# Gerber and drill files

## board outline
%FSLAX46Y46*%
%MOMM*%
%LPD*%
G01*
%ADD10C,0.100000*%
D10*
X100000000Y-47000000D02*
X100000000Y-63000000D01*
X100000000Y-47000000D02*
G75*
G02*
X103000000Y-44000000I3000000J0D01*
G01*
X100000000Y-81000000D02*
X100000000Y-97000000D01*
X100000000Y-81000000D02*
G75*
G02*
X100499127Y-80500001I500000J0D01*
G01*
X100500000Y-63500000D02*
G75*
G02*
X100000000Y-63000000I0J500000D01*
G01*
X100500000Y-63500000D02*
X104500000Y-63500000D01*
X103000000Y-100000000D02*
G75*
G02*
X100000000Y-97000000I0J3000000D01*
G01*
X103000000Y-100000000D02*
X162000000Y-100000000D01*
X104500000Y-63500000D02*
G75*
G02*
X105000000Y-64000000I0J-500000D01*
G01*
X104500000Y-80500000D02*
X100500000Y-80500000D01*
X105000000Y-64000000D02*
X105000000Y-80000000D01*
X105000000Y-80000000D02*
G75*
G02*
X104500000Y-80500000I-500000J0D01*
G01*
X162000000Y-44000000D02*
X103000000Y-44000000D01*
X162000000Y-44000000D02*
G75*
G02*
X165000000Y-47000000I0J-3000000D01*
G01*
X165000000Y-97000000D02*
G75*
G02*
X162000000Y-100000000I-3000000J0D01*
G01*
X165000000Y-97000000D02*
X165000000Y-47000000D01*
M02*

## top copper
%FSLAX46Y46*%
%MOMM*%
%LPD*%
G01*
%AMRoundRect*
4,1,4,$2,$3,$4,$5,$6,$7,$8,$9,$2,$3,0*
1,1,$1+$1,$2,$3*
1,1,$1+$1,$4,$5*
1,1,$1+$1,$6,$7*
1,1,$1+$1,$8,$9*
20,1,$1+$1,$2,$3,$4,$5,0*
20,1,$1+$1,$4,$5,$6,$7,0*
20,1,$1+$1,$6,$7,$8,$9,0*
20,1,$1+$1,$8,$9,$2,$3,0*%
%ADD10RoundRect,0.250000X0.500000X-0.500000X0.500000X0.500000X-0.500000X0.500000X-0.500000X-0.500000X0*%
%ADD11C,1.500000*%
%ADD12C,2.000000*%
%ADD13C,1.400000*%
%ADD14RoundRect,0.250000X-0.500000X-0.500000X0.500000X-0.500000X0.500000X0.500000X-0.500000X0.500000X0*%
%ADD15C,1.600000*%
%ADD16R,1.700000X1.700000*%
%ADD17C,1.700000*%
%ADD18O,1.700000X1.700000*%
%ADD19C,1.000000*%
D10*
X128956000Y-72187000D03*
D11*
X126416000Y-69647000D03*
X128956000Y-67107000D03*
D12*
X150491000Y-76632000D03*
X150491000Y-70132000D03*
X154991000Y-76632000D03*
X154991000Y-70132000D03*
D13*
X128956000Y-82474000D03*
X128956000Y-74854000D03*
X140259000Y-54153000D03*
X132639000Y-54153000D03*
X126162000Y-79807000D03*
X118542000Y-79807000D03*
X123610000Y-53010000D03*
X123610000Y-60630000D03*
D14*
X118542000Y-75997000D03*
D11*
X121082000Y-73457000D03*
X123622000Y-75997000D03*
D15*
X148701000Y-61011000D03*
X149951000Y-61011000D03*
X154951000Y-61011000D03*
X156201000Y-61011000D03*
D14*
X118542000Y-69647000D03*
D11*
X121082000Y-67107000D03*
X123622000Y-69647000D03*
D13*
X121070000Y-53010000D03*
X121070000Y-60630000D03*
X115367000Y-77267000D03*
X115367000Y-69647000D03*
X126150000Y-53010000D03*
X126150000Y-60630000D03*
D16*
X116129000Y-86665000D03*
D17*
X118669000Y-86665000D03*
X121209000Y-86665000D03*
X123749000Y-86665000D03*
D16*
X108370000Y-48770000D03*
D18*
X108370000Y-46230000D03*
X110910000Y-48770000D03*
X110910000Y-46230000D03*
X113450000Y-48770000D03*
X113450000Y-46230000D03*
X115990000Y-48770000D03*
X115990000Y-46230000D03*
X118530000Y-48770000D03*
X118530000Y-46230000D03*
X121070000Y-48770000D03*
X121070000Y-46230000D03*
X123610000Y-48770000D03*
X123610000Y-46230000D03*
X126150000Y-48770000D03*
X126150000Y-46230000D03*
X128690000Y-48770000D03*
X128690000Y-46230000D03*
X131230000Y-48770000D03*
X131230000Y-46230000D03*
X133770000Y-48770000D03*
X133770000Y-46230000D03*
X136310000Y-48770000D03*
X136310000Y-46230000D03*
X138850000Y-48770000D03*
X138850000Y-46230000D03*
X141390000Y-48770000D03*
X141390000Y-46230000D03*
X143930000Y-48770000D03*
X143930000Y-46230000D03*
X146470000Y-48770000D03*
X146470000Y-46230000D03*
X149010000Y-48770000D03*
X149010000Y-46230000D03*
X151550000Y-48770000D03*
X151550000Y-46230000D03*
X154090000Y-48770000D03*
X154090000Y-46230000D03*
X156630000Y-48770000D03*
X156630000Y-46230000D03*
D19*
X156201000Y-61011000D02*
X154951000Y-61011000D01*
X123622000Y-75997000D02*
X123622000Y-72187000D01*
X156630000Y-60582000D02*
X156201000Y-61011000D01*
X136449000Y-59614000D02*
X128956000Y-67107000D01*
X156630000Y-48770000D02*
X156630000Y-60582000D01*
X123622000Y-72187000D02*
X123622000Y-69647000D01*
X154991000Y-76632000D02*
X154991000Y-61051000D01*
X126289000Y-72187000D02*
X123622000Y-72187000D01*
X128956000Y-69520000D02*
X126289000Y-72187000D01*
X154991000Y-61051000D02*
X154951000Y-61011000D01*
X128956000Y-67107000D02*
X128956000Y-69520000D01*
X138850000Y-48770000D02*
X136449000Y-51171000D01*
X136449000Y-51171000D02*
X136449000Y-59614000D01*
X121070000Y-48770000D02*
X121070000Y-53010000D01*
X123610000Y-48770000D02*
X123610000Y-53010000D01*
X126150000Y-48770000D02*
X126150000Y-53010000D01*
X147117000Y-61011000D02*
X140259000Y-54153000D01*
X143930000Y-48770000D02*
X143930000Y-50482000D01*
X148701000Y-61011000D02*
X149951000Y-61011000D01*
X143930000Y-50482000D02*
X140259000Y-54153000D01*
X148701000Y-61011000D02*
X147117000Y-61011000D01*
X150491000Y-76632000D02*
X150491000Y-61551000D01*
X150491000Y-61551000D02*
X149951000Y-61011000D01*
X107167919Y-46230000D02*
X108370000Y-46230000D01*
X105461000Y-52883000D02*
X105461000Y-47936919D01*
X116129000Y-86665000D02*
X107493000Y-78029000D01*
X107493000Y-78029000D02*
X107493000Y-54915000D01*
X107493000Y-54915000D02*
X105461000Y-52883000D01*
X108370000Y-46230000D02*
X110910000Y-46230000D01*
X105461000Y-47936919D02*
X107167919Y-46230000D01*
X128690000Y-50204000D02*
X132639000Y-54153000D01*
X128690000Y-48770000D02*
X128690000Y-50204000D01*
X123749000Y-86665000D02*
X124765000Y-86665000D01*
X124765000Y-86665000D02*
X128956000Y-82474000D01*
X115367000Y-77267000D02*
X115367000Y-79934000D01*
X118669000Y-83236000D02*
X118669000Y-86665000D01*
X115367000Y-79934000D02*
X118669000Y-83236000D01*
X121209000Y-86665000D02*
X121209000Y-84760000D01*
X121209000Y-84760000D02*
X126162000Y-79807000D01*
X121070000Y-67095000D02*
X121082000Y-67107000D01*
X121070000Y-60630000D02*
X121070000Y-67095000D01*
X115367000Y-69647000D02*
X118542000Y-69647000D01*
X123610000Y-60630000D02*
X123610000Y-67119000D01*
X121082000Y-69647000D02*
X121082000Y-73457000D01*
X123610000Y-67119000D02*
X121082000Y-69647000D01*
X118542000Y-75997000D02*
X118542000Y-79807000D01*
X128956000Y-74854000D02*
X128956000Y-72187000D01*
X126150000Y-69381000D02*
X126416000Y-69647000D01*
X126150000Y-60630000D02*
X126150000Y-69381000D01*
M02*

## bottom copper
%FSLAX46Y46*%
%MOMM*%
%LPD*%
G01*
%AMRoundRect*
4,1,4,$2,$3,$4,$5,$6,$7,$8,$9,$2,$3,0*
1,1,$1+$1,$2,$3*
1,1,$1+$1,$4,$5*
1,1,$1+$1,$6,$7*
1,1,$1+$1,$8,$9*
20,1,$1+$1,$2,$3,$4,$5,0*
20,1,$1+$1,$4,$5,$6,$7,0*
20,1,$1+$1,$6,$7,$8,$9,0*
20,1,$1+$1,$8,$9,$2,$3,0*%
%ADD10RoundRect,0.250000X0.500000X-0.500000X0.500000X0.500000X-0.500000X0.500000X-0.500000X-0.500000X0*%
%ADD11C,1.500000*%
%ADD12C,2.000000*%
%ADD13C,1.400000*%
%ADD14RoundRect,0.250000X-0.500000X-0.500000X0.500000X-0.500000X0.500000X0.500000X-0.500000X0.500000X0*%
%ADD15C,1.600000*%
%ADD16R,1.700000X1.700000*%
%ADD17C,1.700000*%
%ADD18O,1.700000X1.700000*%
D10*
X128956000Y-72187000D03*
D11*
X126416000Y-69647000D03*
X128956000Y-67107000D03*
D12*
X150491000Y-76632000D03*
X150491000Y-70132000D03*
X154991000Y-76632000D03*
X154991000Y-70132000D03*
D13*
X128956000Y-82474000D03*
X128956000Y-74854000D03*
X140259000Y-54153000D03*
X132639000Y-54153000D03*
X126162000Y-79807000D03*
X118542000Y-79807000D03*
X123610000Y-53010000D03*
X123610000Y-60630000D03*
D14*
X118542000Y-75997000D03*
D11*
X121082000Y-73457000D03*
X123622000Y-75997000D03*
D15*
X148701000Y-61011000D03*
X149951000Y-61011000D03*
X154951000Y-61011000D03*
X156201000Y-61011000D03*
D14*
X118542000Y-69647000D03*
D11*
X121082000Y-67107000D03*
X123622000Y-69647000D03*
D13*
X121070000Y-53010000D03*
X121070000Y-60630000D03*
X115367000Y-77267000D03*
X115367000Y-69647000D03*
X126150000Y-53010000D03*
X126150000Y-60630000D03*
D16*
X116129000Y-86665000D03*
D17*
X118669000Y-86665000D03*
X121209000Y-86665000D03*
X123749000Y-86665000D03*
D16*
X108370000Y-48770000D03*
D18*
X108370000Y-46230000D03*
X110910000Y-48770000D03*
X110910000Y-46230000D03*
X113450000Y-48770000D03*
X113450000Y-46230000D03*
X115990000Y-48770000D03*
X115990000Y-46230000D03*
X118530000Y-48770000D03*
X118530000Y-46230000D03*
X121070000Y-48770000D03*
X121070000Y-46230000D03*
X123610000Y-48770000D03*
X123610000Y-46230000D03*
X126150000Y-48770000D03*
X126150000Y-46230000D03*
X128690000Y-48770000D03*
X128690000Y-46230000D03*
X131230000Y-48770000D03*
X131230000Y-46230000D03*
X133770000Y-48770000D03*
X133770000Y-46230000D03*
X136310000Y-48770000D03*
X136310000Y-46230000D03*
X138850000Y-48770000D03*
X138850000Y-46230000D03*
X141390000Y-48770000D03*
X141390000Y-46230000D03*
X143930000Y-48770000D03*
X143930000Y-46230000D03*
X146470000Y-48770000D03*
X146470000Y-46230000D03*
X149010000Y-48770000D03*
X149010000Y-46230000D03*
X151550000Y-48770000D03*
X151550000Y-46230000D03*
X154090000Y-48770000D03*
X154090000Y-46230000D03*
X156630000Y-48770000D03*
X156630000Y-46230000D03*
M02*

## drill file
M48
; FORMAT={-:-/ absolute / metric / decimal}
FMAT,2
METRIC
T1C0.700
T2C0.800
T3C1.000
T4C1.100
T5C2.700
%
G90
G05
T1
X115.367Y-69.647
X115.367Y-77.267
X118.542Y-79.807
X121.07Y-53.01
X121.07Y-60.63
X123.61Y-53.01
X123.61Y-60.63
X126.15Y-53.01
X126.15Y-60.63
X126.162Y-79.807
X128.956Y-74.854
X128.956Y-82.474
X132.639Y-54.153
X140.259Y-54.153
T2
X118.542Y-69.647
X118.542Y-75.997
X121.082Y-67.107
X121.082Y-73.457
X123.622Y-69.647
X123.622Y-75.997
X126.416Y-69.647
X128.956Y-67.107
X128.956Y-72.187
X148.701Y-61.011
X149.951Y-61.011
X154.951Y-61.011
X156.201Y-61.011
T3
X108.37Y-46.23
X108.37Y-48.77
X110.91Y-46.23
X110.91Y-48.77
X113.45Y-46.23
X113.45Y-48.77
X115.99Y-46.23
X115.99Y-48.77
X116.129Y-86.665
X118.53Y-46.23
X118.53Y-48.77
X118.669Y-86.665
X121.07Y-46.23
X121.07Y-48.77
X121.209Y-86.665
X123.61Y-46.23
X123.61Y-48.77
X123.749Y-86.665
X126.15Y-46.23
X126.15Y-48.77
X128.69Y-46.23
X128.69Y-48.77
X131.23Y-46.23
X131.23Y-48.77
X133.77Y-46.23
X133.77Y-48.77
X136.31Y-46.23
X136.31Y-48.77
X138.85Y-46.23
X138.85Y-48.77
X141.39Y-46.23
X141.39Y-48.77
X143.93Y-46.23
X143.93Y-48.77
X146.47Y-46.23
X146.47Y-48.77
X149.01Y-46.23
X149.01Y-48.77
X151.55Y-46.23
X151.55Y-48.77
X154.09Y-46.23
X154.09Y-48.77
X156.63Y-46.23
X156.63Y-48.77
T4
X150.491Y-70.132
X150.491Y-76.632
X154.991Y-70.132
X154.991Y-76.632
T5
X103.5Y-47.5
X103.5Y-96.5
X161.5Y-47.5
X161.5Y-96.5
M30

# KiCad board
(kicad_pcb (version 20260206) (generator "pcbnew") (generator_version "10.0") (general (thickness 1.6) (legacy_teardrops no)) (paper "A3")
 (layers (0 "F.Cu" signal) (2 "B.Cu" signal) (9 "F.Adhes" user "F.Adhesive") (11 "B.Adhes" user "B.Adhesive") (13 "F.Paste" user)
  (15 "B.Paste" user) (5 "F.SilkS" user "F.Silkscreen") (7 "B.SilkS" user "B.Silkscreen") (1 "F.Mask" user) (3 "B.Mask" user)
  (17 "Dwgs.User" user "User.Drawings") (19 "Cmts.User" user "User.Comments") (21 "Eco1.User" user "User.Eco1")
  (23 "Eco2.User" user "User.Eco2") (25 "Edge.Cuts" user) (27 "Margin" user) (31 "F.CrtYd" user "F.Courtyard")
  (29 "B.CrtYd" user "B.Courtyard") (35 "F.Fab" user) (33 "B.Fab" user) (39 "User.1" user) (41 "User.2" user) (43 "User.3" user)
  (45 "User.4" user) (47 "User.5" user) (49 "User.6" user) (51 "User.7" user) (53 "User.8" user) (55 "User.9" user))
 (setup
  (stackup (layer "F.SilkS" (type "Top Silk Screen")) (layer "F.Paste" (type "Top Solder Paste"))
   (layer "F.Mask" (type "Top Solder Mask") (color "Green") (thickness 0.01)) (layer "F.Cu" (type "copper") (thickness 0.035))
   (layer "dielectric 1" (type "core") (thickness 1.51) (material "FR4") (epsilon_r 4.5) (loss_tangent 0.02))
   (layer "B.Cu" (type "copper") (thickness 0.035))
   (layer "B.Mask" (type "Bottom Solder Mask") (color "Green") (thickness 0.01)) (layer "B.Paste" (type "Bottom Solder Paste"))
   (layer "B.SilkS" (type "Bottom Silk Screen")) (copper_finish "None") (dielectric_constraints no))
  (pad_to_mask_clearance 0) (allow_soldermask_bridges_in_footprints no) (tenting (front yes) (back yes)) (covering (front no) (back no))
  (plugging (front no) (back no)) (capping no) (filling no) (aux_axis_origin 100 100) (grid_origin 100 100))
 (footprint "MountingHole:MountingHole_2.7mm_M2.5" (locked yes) (layer "F.Cu") (at 161.5 47.5)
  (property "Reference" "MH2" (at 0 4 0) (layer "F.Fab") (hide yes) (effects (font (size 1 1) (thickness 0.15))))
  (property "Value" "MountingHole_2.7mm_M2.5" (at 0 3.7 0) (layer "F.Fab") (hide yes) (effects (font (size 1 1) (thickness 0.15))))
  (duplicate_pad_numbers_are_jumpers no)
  (pad "" np_thru_hole circle (at 0 0) (size 2.7 2.7) (drill 2.7) (layers "*.Cu" "*.Mask")))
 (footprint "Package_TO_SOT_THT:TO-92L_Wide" (layer "F.Cu") (at 128.956 72.187 90)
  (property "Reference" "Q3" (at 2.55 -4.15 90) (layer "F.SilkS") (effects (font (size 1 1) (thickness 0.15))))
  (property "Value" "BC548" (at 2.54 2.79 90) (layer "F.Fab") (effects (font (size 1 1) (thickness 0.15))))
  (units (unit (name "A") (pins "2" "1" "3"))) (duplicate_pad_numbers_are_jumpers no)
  (pad "1" thru_hole roundrect (at 0 0 90) (size 1.5 1.5) (drill 0.8) (layers "*.Cu" "*.Mask") (remove_unused_layers no)
   (roundrect_rratio 0.1666666667) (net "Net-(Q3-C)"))
  (pad "2" thru_hole circle (at 2.54 -2.54 90) (size 1.5 1.5) (drill 0.8) (layers "*.Cu" "*.Mask") (remove_unused_layers no)
   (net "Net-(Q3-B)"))
  (pad "3" thru_hole circle (at 5.08 0 90) (size 1.5 1.5) (drill 0.8) (layers "*.Cu" "*.Mask") (remove_unused_layers no) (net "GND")))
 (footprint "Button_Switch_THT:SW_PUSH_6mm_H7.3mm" (layer "F.Cu") (at 150.491 76.632 90)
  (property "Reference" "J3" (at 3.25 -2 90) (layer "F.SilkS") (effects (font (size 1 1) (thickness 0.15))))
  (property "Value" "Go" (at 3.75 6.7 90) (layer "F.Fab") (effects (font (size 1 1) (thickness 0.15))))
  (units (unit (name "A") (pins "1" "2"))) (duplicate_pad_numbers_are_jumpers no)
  (pad "1" thru_hole circle (at 0 0 180) (size 2 2) (drill 1.1) (layers "*.Cu" "*.Mask") (remove_unused_layers no) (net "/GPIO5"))
  (pad "1" thru_hole circle (at 6.5 0 180) (size 2 2) (drill 1.1) (layers "*.Cu" "*.Mask") (remove_unused_layers no) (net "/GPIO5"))
  (pad "2" thru_hole circle (at 0 4.5 180) (size 2 2) (drill 1.1) (layers "*.Cu" "*.Mask") (remove_unused_layers no) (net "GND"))
  (pad "2" thru_hole circle (at 6.5 4.5 180) (size 2 2) (drill 1.1) (layers "*.Cu" "*.Mask") (remove_unused_layers no) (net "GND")))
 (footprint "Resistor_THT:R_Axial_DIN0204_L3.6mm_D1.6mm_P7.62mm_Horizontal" (layer "F.Cu") (at 128.956 82.474 90)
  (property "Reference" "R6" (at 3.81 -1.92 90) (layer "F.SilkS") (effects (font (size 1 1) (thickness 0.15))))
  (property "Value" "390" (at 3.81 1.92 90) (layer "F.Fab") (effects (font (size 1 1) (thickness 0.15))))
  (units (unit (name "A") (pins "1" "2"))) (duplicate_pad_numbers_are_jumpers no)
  (pad "1" thru_hole circle (at 0 0 90) (size 1.4 1.4) (drill 0.7) (layers "*.Cu" "*.Mask") (remove_unused_layers no) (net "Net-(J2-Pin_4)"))
  (pad "2" thru_hole circle (at 7.62 0 90) (size 1.4 1.4) (drill 0.7) (layers "*.Cu" "*.Mask") (remove_unused_layers no) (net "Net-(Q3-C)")))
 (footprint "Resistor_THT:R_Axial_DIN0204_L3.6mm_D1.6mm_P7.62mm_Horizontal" (layer "F.Cu") (at 140.259 54.153 180)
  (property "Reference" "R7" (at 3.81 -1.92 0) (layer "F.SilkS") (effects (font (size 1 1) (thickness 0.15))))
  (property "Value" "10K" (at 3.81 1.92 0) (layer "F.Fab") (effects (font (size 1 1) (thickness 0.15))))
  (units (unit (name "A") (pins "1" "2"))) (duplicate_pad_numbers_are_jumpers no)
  (pad "1" thru_hole circle (at 0 0 180) (size 1.4 1.4) (drill 0.7) (layers "*.Cu" "*.Mask") (remove_unused_layers no) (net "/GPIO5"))
  (pad "2" thru_hole circle (at 7.62 0 180) (size 1.4 1.4) (drill 0.7) (layers "*.Cu" "*.Mask") (remove_unused_layers no) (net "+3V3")))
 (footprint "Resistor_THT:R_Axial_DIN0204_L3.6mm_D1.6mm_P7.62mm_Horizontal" (layer "F.Cu") (at 126.162 79.807 180)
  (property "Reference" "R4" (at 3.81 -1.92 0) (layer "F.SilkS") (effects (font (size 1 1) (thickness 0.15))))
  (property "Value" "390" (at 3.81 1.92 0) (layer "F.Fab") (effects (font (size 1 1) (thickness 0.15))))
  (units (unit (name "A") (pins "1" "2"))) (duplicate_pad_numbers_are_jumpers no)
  (pad "1" thru_hole circle (at 0 0 180) (size 1.4 1.4) (drill 0.7) (layers "*.Cu" "*.Mask") (remove_unused_layers no)
   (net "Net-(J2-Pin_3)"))
  (pad "2" thru_hole circle (at 7.62 0 180) (size 1.4 1.4) (drill 0.7) (layers "*.Cu" "*.Mask") (remove_unused_layers no) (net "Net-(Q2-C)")))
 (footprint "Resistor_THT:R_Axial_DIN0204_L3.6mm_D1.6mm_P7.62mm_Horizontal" (layer "F.Cu") (at 123.61 53.01 -90)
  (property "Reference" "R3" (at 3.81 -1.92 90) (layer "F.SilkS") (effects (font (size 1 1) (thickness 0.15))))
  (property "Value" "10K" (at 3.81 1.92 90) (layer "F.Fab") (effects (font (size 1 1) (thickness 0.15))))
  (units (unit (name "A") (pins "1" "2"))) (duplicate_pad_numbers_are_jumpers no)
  (pad "1" thru_hole circle (at 0 0 270) (size 1.4 1.4) (drill 0.7) (layers "*.Cu" "*.Mask") (remove_unused_layers no) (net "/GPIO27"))
  (pad "2" thru_hole circle (at 7.62 0 270) (size 1.4 1.4) (drill 0.7) (layers "*.Cu" "*.Mask") (remove_unused_layers no) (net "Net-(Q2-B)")))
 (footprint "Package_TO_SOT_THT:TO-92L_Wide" (layer "F.Cu") (at 118.542 75.997)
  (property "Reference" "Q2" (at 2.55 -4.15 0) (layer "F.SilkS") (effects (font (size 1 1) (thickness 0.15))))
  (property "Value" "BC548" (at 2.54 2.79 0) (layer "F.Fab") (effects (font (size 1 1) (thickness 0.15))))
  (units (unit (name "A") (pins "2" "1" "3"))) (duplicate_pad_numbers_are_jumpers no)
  (pad "1" thru_hole roundrect (at 0 0) (size 1.5 1.5) (drill 0.8) (layers "*.Cu" "*.Mask") (remove_unused_layers no)
   (roundrect_rratio 0.1666666667) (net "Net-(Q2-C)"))
  (pad "2" thru_hole circle (at 2.54 -2.54) (size 1.5 1.5) (drill 0.8) (layers "*.Cu" "*.Mask") (remove_unused_layers no) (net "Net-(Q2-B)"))
  (pad "3" thru_hole circle (at 5.08 0) (size 1.5 1.5) (drill 0.8) (layers "*.Cu" "*.Mask") (remove_unused_layers no) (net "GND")))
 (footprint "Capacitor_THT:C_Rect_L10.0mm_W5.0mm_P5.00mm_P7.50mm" (layer "F.Cu") (at 148.701 61.011)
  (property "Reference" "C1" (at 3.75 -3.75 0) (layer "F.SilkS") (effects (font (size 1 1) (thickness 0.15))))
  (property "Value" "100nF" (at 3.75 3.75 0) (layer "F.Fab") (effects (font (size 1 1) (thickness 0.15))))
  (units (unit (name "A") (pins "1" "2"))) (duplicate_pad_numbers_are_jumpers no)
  (pad "1" thru_hole circle (at 0 0) (size 1.6 1.6) (drill 0.8) (layers "*.Cu" "*.Mask") (remove_unused_layers no) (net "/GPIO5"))
  (pad "1" thru_hole circle (at 1.25 0) (size 1.6 1.6) (drill 0.8) (layers "*.Cu" "*.Mask") (remove_unused_layers no) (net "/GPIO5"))
  (pad "2" thru_hole circle (at 6.25 0) (size 1.6 1.6) (drill 0.8) (layers "*.Cu" "*.Mask") (remove_unused_layers no) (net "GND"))
  (pad "2" thru_hole circle (at 7.5 0) (size 1.6 1.6) (drill 0.8) (layers "*.Cu" "*.Mask") (remove_unused_layers no) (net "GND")))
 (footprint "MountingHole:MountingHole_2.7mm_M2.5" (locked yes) (layer "F.Cu") (at 103.5 96.5)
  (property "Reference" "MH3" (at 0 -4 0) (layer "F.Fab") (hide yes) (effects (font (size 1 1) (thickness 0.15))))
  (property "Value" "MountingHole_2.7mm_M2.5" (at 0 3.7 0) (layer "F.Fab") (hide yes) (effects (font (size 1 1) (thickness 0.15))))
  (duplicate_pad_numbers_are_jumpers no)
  (pad "" np_thru_hole circle (at 0 0) (size 2.7 2.7) (drill 2.7) (layers "*.Cu" "*.Mask")))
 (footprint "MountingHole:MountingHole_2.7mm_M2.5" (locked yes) (layer "F.Cu") (at 103.5 47.5)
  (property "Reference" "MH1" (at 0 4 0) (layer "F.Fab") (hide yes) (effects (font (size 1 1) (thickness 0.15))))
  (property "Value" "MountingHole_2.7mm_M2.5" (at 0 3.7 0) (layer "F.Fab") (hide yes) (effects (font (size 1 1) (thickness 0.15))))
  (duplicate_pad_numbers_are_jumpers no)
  (pad "" np_thru_hole circle (at 0 0) (size 2.7 2.7) (drill 2.7) (layers "*.Cu" "*.Mask")))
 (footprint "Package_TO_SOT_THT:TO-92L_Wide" (layer "F.Cu") (at 118.542 69.647)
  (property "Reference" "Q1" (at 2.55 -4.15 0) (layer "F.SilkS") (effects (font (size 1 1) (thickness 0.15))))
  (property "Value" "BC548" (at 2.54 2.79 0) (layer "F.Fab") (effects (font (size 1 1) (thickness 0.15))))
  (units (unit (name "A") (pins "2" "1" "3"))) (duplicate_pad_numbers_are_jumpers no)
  (pad "1" thru_hole roundrect (at 0 0) (size 1.5 1.5) (drill 0.8) (layers "*.Cu" "*.Mask") (remove_unused_layers no)
   (roundrect_rratio 0.1666666667) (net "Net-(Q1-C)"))
  (pad "2" thru_hole circle (at 2.54 -2.54) (size 1.5 1.5) (drill 0.8) (layers "*.Cu" "*.Mask") (remove_unused_layers no) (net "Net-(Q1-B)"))
  (pad "3" thru_hole circle (at 5.08 0) (size 1.5 1.5) (drill 0.8) (layers "*.Cu" "*.Mask") (remove_unused_layers no) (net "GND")))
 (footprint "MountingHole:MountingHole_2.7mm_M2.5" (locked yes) (layer "F.Cu") (at 161.5 96.5)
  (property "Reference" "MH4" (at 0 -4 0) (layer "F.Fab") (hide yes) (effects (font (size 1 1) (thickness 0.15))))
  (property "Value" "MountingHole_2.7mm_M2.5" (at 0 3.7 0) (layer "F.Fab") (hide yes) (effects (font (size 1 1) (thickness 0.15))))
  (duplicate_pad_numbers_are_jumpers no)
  (pad "" np_thru_hole circle (at 0 0) (size 2.7 2.7) (drill 2.7) (layers "*.Cu" "*.Mask")))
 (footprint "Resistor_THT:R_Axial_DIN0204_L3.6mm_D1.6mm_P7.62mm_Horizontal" (layer "F.Cu") (at 121.07 53.01 -90)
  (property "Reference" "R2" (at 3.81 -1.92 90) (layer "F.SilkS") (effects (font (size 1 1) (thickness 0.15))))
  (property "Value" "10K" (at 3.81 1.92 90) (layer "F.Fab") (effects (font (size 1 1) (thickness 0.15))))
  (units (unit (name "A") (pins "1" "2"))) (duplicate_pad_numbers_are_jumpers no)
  (pad "1" thru_hole circle (at 0 0 270) (size 1.4 1.4) (drill 0.7) (layers "*.Cu" "*.Mask") (remove_unused_layers no) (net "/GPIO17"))
  (pad "2" thru_hole circle (at 7.62 0 270) (size 1.4 1.4) (drill 0.7) (layers "*.Cu" "*.Mask") (remove_unused_layers no) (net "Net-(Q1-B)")))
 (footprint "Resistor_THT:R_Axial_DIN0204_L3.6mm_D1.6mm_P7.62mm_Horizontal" (layer "F.Cu") (at 115.367 77.267 90)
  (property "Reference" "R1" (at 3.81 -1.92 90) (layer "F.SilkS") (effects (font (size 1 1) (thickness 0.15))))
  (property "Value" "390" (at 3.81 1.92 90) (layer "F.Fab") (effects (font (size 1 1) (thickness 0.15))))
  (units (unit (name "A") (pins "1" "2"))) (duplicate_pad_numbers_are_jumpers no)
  (pad "1" thru_hole circle (at 0 0 90) (size 1.4 1.4) (drill 0.7) (layers "*.Cu" "*.Mask") (remove_unused_layers no) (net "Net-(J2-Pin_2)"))
  (pad "2" thru_hole circle (at 7.62 0 90) (size 1.4 1.4) (drill 0.7) (layers "*.Cu" "*.Mask") (remove_unused_layers no) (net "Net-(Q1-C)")))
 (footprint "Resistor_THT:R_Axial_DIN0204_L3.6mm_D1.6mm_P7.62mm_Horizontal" (layer "F.Cu") (at 126.15 53.01 -90)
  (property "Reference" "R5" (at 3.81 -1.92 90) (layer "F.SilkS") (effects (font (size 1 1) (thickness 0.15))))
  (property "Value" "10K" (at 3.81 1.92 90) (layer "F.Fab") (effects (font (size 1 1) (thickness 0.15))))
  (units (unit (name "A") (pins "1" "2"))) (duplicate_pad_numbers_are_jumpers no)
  (pad "1" thru_hole circle (at 0 0 270) (size 1.4 1.4) (drill 0.7) (layers "*.Cu" "*.Mask") (remove_unused_layers no) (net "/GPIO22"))
  (pad "2" thru_hole circle (at 7.62 0 270) (size 1.4 1.4) (drill 0.7) (layers "*.Cu" "*.Mask") (remove_unused_layers no) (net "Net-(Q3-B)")))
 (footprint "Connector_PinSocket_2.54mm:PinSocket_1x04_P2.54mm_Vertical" (layer "F.Cu") (at 116.129 86.665 90)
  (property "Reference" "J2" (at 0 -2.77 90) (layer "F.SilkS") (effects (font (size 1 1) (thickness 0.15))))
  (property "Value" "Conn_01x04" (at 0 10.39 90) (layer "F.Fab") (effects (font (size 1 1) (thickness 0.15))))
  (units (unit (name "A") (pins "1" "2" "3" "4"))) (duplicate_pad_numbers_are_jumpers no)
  (pad "1" thru_hole rect (at 0 0 90) (size 1.7 1.7) (drill 1) (layers "*.Cu" "*.Mask") (remove_unused_layers no) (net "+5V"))
  (pad "2" thru_hole circle (at 0 2.54 90) (size 1.7 1.7) (drill 1) (layers "*.Cu" "*.Mask") (remove_unused_layers no)
   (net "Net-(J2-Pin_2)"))
  (pad "3" thru_hole circle (at 0 5.08 90) (size 1.7 1.7) (drill 1) (layers "*.Cu" "*.Mask") (remove_unused_layers no)
   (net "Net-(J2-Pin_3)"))
  (pad "4" thru_hole circle (at 0 7.62 90) (size 1.7 1.7) (drill 1) (layers "*.Cu" "*.Mask") (remove_unused_layers no)
   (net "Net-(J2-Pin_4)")))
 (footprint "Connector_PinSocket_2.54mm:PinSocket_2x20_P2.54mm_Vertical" (layer "B.Cu") (at 108.37 48.77 -90)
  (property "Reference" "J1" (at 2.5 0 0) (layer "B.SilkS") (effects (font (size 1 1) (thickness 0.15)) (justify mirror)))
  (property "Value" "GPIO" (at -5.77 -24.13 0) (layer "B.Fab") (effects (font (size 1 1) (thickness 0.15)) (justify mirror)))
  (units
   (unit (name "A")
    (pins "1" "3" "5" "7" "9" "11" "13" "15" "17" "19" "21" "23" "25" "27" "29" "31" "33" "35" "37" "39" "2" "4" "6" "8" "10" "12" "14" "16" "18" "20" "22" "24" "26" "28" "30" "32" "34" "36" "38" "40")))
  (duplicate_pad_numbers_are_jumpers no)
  (pad "1" thru_hole rect (at 0 0 270) (size 1.7 1.7) (drill 1) (layers "*.Cu" "*.Mask") (remove_unused_layers no) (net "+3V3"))
  (pad "2" thru_hole oval (at -2.54 0 270) (size 1.7 1.7) (drill 1) (layers "*.Cu" "*.Mask") (remove_unused_layers no) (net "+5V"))
  (pad "3" thru_hole oval (at 0 -2.54 270) (size 1.7 1.7) (drill 1) (layers "*.Cu" "*.Mask") (remove_unused_layers no)
   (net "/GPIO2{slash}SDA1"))
  (pad "4" thru_hole oval (at -2.54 -2.54 270) (size 1.7 1.7) (drill 1) (layers "*.Cu" "*.Mask") (remove_unused_layers no) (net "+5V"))
  (pad "5" thru_hole oval (at 0 -5.08 270) (size 1.7 1.7) (drill 1) (layers "*.Cu" "*.Mask") (remove_unused_layers no)
   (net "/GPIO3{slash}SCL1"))
  (pad "6" thru_hole oval (at -2.54 -5.08 270) (size 1.7 1.7) (drill 1) (layers "*.Cu" "*.Mask") (remove_unused_layers no) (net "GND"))
  (pad "7" thru_hole oval (at 0 -7.62 270) (size 1.7 1.7) (drill 1) (layers "*.Cu" "*.Mask") (remove_unused_layers no)
   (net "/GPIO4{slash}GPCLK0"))
  (pad "8" thru_hole oval (at -2.54 -7.62 270) (size 1.7 1.7) (drill 1) (layers "*.Cu" "*.Mask") (remove_unused_layers no)
   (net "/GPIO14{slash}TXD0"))
  (pad "9" thru_hole oval (at 0 -10.16 270) (size 1.7 1.7) (drill 1) (layers "*.Cu" "*.Mask") (remove_unused_layers no) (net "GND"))
  (pad "10" thru_hole oval (at -2.54 -10.16 270) (size 1.7 1.7) (drill 1) (layers "*.Cu" "*.Mask") (remove_unused_layers no)
   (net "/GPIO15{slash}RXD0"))
  (pad "11" thru_hole oval (at 0 -12.7 270) (size 1.7 1.7) (drill 1) (layers "*.Cu" "*.Mask") (remove_unused_layers no) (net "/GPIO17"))
  (pad "12" thru_hole oval (at -2.54 -12.7 270) (size 1.7 1.7) (drill 1) (layers "*.Cu" "*.Mask") (remove_unused_layers no)
   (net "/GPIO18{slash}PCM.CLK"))
  (pad "13" thru_hole oval (at 0 -15.24 270) (size 1.7 1.7) (drill 1) (layers "*.Cu" "*.Mask") (remove_unused_layers no) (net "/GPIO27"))
  (pad "14" thru_hole oval (at -2.54 -15.24 270) (size 1.7 1.7) (drill 1) (layers "*.Cu" "*.Mask") (remove_unused_layers no) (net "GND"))
  (pad "15" thru_hole oval (at 0 -17.78 270) (size 1.7 1.7) (drill 1) (layers "*.Cu" "*.Mask") (remove_unused_layers no) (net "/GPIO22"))
  (pad "16" thru_hole oval (at -2.54 -17.78 270) (size 1.7 1.7) (drill 1) (layers "*.Cu" "*.Mask") (remove_unused_layers no) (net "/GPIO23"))
  (pad "17" thru_hole oval (at 0 -20.32 270) (size 1.7 1.7) (drill 1) (layers "*.Cu" "*.Mask") (remove_unused_layers no) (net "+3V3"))
  (pad "18" thru_hole oval (at -2.54 -20.32 270) (size 1.7 1.7) (drill 1) (layers "*.Cu" "*.Mask") (remove_unused_layers no) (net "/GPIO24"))
  (pad "19" thru_hole oval (at 0 -22.86 270) (size 1.7 1.7) (drill 1) (layers "*.Cu" "*.Mask") (remove_unused_layers no)
   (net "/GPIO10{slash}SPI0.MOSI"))
  (pad "20" thru_hole oval (at -2.54 -22.86 270) (size 1.7 1.7) (drill 1) (layers "*.Cu" "*.Mask") (remove_unused_layers no) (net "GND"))
  (pad "21" thru_hole oval (at 0 -25.4 270) (size 1.7 1.7) (drill 1) (layers "*.Cu" "*.Mask") (remove_unused_layers no)
   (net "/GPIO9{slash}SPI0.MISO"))
  (pad "22" thru_hole oval (at -2.54 -25.4 270) (size 1.7 1.7) (drill 1) (layers "*.Cu" "*.Mask") (remove_unused_layers no) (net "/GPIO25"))
  (pad "23" thru_hole oval (at 0 -27.94 270) (size 1.7 1.7) (drill 1) (layers "*.Cu" "*.Mask") (remove_unused_layers no)
   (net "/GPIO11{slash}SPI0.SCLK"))
  (pad "24" thru_hole oval (at -2.54 -27.94 270) (size 1.7 1.7) (drill 1) (layers "*.Cu" "*.Mask") (remove_unused_layers no)
   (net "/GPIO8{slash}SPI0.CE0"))
  (pad "25" thru_hole oval (at 0 -30.48 270) (size 1.7 1.7) (drill 1) (layers "*.Cu" "*.Mask") (remove_unused_layers no) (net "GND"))
  (pad "26" thru_hole oval (at -2.54 -30.48 270) (size 1.7 1.7) (drill 1) (layers "*.Cu" "*.Mask") (remove_unused_layers no)
   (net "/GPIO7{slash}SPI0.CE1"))
  (pad "27" thru_hole oval (at 0 -33.02 270) (size 1.7 1.7) (drill 1) (layers "*.Cu" "*.Mask") (remove_unused_layers no) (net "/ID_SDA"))
  (pad "28" thru_hole oval (at -2.54 -33.02 270) (size 1.7 1.7) (drill 1) (layers "*.Cu" "*.Mask") (remove_unused_layers no) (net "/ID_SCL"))
  (pad "29" thru_hole oval (at 0 -35.56 270) (size 1.7 1.7) (drill 1) (layers "*.Cu" "*.Mask") (remove_unused_layers no) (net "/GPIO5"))
  (pad "30" thru_hole oval (at -2.54 -35.56 270) (size 1.7 1.7) (drill 1) (layers "*.Cu" "*.Mask") (remove_unused_layers no) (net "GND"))
  (pad "31" thru_hole oval (at 0 -38.1 270) (size 1.7 1.7) (drill 1) (layers "*.Cu" "*.Mask") (remove_unused_layers no) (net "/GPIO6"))
  (pad "32" thru_hole oval (at -2.54 -38.1 270) (size 1.7 1.7) (drill 1) (layers "*.Cu" "*.Mask") (remove_unused_layers no)
   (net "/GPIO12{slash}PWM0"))
  (pad "33" thru_hole oval (at 0 -40.64 270) (size 1.7 1.7) (drill 1) (layers "*.Cu" "*.Mask") (remove_unused_layers no)
   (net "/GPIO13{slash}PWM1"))
  (pad "34" thru_hole oval (at -2.54 -40.64 270) (size 1.7 1.7) (drill 1) (layers "*.Cu" "*.Mask") (remove_unused_layers no) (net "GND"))
  (pad "35" thru_hole oval (at 0 -43.18 270) (size 1.7 1.7) (drill 1) (layers "*.Cu" "*.Mask") (remove_unused_layers no)
   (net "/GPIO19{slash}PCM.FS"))
  (pad "36" thru_hole oval (at -2.54 -43.18 270) (size 1.7 1.7) (drill 1) (layers "*.Cu" "*.Mask") (remove_unused_layers no) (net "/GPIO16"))
  (pad "37" thru_hole oval (at 0 -45.72 270) (size 1.7 1.7) (drill 1) (layers "*.Cu" "*.Mask") (remove_unused_layers no) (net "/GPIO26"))
  (pad "38" thru_hole oval (at -2.54 -45.72 270) (size 1.7 1.7) (drill 1) (layers "*.Cu" "*.Mask") (remove_unused_layers no)
   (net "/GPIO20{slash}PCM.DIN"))
  (pad "39" thru_hole oval (at 0 -48.26 270) (size 1.7 1.7) (drill 1) (layers "*.Cu" "*.Mask") (remove_unused_layers no) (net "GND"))
  (pad "40" thru_hole oval (at -2.54 -48.26 270) (size 1.7 1.7) (drill 1) (layers "*.Cu" "*.Mask") (remove_unused_layers no)
   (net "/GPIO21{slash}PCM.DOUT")))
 (gr_line (start 100 47) (end 100 63) (stroke (width 0.1) (type solid)) (layer "Edge.Cuts"))
 (gr_arc (start 100 47) (mid 100.87868 44.87868) (end 103 44) (stroke (width 0.1) (type solid)) (layer "Edge.Cuts"))
 (gr_line (start 100 81) (end 100 97) (stroke (width 0.1) (type solid)) (layer "Edge.Cuts"))
 (gr_arc (start 100 81) (mid 100.146138 80.646755) (end 100.499127 80.500001) (stroke (width 0.1) (type solid)) (layer "Edge.Cuts"))
 (gr_arc (start 100.5 63.5) (mid 100.146447 63.353553) (end 100 63) (stroke (width 0.1) (type solid)) (layer "Edge.Cuts"))
 (gr_line (start 100.5 63.5) (end 104.5 63.5) (stroke (width 0.1) (type solid)) (layer "Edge.Cuts"))
 (gr_arc (start 103 100) (mid 100.87868 99.12132) (end 100 97) (stroke (width 0.1) (type solid)) (layer "Edge.Cuts"))
 (gr_line (start 103 100) (end 162 100) (stroke (width 0.1) (type solid)) (layer "Edge.Cuts"))
 (gr_arc (start 104.5 63.5) (mid 104.853553 63.646447) (end 105 64) (stroke (width 0.1) (type solid)) (layer "Edge.Cuts"))
 (gr_line (start 104.5 80.5) (end 100.5 80.5) (stroke (width 0.1) (type solid)) (layer "Edge.Cuts"))
 (gr_line (start 105 64) (end 105 80) (stroke (width 0.1) (type solid)) (layer "Edge.Cuts"))
 (gr_arc (start 105 80) (mid 104.853553 80.353553) (end 104.5 80.5) (stroke (width 0.1) (type solid)) (layer "Edge.Cuts"))
 (gr_line (start 162 44) (end 103 44) (stroke (width 0.1) (type solid)) (layer "Edge.Cuts"))
 (gr_arc (start 162 44) (mid 164.12132 44.87868) (end 165 47) (stroke (width 0.1) (type solid)) (layer "Edge.Cuts"))
 (gr_arc (start 165 97) (mid 164.12132 99.12132) (end 162 100) (stroke (width 0.1) (type solid)) (layer "Edge.Cuts"))
 (gr_line (start 165 97) (end 165 47) (stroke (width 0.1) (type solid)) (layer "Edge.Cuts"))
 (segment (start 156.201 61.011) (end 154.951 61.011) (width 1) (layer "F.Cu") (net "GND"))
 (segment (start 123.622 75.997) (end 123.622 72.187) (width 1) (layer "F.Cu") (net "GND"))
 (segment (start 156.63 60.582) (end 156.201 61.011) (width 1) (layer "F.Cu") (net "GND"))
 (segment (start 136.449 59.614) (end 128.956 67.107) (width 1) (layer "F.Cu") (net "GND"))
 (segment (start 156.63 48.77) (end 156.63 60.582) (width 1) (layer "F.Cu") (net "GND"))
 (segment (start 123.622 72.187) (end 123.622 69.647) (width 1) (layer "F.Cu") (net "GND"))
 (segment (start 154.991 76.632) (end 154.991 61.051) (width 1) (layer "F.Cu") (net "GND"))
 (segment (start 126.289 72.187) (end 123.622 72.187) (width 1) (layer "F.Cu") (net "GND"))
 (segment (start 128.956 69.52) (end 126.289 72.187) (width 1) (layer "F.Cu") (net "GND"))
 (segment (start 154.991 61.051) (end 154.951 61.011) (width 1) (layer "F.Cu") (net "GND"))
 (segment (start 128.956 67.107) (end 128.956 69.52) (width 1) (layer "F.Cu") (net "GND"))
 (segment (start 138.85 48.77) (end 136.449 51.171) (width 1) (layer "F.Cu") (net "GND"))
 (segment (start 136.449 51.171) (end 136.449 59.614) (width 1) (layer "F.Cu") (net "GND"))
 (segment (start 121.07 48.77) (end 121.07 53.01) (width 1) (layer "F.Cu") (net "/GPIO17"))
 (segment (start 123.61 48.77) (end 123.61 53.01) (width 1) (layer "F.Cu") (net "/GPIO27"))
 (segment (start 126.15 48.77) (end 126.15 53.01) (width 1) (layer "F.Cu") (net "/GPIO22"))
 (segment (start 147.117 61.011) (end 140.259 54.153) (width 1) (layer "F.Cu") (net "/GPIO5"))
 (segment (start 143.93 48.77) (end 143.93 50.482) (width 1) (layer "F.Cu") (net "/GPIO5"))
 (segment (start 148.701 61.011) (end 149.951 61.011) (width 1) (layer "F.Cu") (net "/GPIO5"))
 (segment (start 143.93 50.482) (end 140.259 54.153) (width 1) (layer "F.Cu") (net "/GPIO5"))
 (segment (start 148.701 61.011) (end 147.117 61.011) (width 1) (layer "F.Cu") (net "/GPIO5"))
 (segment (start 150.491 76.632) (end 150.491 61.551) (width 1) (layer "F.Cu") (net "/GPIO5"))
 (segment (start 150.491 61.551) (end 149.951 61.011) (width 1) (layer "F.Cu") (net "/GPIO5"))
 (segment (start 107.167919 46.23) (end 108.37 46.23) (width 1) (layer "F.Cu") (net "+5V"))
 (segment (start 105.461 52.883) (end 105.461 47.936919) (width 1) (layer "F.Cu") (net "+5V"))
 (segment (start 116.129 86.665) (end 107.493 78.029) (width 1) (layer "F.Cu") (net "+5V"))
 (segment (start 107.493 78.029) (end 107.493 54.915) (width 1) (layer "F.Cu") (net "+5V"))
 (segment (start 107.493 54.915) (end 105.461 52.883) (width 1) (layer "F.Cu") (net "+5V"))
 (segment (start 108.37 46.23) (end 110.91 46.23) (width 1) (layer "F.Cu") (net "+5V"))
 (segment (start 105.461 47.936919) (end 107.167919 46.23) (width 1) (layer "F.Cu") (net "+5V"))
 (segment (start 128.69 50.204) (end 132.639 54.153) (width 1) (layer "F.Cu") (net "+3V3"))
 (segment (start 128.69 48.77) (end 128.69 50.204) (width 1) (layer "F.Cu") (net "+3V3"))
 (segment (start 123.749 86.665) (end 124.765 86.665) (width 1) (layer "F.Cu") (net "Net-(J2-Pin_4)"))
 (segment (start 124.765 86.665) (end 128.956 82.474) (width 1) (layer "F.Cu") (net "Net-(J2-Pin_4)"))
 (segment (start 115.367 77.267) (end 115.367 79.934) (width 1) (layer "F.Cu") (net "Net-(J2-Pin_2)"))
 (segment (start 118.669 83.236) (end 118.669 86.665) (width 1) (layer "F.Cu") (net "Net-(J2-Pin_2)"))
 (segment (start 115.367 79.934) (end 118.669 83.236) (width 1) (layer "F.Cu") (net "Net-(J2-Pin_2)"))
 (segment (start 121.209 86.665) (end 121.209 84.76) (width 1) (layer "F.Cu") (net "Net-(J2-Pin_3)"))
 (segment (start 121.209 84.76) (end 126.162 79.807) (width 1) (layer "F.Cu") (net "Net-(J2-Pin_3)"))
 (segment (start 121.07 67.095) (end 121.082 67.107) (width 1) (layer "F.Cu") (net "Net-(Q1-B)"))
 (segment (start 121.07 60.63) (end 121.07 67.095) (width 1) (layer "F.Cu") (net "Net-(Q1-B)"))
 (segment (start 115.367 69.647) (end 118.542 69.647) (width 1) (layer "F.Cu") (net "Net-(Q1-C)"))
 (segment (start 123.61 60.63) (end 123.61 67.119) (width 1) (layer "F.Cu") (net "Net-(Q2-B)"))
 (segment (start 121.082 69.647) (end 121.082 73.457) (width 1) (layer "F.Cu") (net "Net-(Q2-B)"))
 (segment (start 123.61 67.119) (end 121.082 69.647) (width 1) (layer "F.Cu") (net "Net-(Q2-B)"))
 (segment (start 118.542 75.997) (end 118.542 79.807) (width 1) (layer "F.Cu") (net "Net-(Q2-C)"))
 (segment (start 128.956 74.854) (end 128.956 72.187) (width 1) (layer "F.Cu") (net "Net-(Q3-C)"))
 (segment (start 126.15 69.381) (end 126.416 69.647) (width 1) (layer "F.Cu") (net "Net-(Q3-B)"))
 (segment (start 126.15 60.63) (end 126.15 69.381) (width 1) (layer "F.Cu") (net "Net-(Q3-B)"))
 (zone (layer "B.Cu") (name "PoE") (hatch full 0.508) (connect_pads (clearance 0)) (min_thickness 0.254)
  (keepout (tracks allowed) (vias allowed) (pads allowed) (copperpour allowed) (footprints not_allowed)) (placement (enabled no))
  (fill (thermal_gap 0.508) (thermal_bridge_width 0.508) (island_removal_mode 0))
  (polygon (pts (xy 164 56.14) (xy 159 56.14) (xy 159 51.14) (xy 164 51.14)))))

